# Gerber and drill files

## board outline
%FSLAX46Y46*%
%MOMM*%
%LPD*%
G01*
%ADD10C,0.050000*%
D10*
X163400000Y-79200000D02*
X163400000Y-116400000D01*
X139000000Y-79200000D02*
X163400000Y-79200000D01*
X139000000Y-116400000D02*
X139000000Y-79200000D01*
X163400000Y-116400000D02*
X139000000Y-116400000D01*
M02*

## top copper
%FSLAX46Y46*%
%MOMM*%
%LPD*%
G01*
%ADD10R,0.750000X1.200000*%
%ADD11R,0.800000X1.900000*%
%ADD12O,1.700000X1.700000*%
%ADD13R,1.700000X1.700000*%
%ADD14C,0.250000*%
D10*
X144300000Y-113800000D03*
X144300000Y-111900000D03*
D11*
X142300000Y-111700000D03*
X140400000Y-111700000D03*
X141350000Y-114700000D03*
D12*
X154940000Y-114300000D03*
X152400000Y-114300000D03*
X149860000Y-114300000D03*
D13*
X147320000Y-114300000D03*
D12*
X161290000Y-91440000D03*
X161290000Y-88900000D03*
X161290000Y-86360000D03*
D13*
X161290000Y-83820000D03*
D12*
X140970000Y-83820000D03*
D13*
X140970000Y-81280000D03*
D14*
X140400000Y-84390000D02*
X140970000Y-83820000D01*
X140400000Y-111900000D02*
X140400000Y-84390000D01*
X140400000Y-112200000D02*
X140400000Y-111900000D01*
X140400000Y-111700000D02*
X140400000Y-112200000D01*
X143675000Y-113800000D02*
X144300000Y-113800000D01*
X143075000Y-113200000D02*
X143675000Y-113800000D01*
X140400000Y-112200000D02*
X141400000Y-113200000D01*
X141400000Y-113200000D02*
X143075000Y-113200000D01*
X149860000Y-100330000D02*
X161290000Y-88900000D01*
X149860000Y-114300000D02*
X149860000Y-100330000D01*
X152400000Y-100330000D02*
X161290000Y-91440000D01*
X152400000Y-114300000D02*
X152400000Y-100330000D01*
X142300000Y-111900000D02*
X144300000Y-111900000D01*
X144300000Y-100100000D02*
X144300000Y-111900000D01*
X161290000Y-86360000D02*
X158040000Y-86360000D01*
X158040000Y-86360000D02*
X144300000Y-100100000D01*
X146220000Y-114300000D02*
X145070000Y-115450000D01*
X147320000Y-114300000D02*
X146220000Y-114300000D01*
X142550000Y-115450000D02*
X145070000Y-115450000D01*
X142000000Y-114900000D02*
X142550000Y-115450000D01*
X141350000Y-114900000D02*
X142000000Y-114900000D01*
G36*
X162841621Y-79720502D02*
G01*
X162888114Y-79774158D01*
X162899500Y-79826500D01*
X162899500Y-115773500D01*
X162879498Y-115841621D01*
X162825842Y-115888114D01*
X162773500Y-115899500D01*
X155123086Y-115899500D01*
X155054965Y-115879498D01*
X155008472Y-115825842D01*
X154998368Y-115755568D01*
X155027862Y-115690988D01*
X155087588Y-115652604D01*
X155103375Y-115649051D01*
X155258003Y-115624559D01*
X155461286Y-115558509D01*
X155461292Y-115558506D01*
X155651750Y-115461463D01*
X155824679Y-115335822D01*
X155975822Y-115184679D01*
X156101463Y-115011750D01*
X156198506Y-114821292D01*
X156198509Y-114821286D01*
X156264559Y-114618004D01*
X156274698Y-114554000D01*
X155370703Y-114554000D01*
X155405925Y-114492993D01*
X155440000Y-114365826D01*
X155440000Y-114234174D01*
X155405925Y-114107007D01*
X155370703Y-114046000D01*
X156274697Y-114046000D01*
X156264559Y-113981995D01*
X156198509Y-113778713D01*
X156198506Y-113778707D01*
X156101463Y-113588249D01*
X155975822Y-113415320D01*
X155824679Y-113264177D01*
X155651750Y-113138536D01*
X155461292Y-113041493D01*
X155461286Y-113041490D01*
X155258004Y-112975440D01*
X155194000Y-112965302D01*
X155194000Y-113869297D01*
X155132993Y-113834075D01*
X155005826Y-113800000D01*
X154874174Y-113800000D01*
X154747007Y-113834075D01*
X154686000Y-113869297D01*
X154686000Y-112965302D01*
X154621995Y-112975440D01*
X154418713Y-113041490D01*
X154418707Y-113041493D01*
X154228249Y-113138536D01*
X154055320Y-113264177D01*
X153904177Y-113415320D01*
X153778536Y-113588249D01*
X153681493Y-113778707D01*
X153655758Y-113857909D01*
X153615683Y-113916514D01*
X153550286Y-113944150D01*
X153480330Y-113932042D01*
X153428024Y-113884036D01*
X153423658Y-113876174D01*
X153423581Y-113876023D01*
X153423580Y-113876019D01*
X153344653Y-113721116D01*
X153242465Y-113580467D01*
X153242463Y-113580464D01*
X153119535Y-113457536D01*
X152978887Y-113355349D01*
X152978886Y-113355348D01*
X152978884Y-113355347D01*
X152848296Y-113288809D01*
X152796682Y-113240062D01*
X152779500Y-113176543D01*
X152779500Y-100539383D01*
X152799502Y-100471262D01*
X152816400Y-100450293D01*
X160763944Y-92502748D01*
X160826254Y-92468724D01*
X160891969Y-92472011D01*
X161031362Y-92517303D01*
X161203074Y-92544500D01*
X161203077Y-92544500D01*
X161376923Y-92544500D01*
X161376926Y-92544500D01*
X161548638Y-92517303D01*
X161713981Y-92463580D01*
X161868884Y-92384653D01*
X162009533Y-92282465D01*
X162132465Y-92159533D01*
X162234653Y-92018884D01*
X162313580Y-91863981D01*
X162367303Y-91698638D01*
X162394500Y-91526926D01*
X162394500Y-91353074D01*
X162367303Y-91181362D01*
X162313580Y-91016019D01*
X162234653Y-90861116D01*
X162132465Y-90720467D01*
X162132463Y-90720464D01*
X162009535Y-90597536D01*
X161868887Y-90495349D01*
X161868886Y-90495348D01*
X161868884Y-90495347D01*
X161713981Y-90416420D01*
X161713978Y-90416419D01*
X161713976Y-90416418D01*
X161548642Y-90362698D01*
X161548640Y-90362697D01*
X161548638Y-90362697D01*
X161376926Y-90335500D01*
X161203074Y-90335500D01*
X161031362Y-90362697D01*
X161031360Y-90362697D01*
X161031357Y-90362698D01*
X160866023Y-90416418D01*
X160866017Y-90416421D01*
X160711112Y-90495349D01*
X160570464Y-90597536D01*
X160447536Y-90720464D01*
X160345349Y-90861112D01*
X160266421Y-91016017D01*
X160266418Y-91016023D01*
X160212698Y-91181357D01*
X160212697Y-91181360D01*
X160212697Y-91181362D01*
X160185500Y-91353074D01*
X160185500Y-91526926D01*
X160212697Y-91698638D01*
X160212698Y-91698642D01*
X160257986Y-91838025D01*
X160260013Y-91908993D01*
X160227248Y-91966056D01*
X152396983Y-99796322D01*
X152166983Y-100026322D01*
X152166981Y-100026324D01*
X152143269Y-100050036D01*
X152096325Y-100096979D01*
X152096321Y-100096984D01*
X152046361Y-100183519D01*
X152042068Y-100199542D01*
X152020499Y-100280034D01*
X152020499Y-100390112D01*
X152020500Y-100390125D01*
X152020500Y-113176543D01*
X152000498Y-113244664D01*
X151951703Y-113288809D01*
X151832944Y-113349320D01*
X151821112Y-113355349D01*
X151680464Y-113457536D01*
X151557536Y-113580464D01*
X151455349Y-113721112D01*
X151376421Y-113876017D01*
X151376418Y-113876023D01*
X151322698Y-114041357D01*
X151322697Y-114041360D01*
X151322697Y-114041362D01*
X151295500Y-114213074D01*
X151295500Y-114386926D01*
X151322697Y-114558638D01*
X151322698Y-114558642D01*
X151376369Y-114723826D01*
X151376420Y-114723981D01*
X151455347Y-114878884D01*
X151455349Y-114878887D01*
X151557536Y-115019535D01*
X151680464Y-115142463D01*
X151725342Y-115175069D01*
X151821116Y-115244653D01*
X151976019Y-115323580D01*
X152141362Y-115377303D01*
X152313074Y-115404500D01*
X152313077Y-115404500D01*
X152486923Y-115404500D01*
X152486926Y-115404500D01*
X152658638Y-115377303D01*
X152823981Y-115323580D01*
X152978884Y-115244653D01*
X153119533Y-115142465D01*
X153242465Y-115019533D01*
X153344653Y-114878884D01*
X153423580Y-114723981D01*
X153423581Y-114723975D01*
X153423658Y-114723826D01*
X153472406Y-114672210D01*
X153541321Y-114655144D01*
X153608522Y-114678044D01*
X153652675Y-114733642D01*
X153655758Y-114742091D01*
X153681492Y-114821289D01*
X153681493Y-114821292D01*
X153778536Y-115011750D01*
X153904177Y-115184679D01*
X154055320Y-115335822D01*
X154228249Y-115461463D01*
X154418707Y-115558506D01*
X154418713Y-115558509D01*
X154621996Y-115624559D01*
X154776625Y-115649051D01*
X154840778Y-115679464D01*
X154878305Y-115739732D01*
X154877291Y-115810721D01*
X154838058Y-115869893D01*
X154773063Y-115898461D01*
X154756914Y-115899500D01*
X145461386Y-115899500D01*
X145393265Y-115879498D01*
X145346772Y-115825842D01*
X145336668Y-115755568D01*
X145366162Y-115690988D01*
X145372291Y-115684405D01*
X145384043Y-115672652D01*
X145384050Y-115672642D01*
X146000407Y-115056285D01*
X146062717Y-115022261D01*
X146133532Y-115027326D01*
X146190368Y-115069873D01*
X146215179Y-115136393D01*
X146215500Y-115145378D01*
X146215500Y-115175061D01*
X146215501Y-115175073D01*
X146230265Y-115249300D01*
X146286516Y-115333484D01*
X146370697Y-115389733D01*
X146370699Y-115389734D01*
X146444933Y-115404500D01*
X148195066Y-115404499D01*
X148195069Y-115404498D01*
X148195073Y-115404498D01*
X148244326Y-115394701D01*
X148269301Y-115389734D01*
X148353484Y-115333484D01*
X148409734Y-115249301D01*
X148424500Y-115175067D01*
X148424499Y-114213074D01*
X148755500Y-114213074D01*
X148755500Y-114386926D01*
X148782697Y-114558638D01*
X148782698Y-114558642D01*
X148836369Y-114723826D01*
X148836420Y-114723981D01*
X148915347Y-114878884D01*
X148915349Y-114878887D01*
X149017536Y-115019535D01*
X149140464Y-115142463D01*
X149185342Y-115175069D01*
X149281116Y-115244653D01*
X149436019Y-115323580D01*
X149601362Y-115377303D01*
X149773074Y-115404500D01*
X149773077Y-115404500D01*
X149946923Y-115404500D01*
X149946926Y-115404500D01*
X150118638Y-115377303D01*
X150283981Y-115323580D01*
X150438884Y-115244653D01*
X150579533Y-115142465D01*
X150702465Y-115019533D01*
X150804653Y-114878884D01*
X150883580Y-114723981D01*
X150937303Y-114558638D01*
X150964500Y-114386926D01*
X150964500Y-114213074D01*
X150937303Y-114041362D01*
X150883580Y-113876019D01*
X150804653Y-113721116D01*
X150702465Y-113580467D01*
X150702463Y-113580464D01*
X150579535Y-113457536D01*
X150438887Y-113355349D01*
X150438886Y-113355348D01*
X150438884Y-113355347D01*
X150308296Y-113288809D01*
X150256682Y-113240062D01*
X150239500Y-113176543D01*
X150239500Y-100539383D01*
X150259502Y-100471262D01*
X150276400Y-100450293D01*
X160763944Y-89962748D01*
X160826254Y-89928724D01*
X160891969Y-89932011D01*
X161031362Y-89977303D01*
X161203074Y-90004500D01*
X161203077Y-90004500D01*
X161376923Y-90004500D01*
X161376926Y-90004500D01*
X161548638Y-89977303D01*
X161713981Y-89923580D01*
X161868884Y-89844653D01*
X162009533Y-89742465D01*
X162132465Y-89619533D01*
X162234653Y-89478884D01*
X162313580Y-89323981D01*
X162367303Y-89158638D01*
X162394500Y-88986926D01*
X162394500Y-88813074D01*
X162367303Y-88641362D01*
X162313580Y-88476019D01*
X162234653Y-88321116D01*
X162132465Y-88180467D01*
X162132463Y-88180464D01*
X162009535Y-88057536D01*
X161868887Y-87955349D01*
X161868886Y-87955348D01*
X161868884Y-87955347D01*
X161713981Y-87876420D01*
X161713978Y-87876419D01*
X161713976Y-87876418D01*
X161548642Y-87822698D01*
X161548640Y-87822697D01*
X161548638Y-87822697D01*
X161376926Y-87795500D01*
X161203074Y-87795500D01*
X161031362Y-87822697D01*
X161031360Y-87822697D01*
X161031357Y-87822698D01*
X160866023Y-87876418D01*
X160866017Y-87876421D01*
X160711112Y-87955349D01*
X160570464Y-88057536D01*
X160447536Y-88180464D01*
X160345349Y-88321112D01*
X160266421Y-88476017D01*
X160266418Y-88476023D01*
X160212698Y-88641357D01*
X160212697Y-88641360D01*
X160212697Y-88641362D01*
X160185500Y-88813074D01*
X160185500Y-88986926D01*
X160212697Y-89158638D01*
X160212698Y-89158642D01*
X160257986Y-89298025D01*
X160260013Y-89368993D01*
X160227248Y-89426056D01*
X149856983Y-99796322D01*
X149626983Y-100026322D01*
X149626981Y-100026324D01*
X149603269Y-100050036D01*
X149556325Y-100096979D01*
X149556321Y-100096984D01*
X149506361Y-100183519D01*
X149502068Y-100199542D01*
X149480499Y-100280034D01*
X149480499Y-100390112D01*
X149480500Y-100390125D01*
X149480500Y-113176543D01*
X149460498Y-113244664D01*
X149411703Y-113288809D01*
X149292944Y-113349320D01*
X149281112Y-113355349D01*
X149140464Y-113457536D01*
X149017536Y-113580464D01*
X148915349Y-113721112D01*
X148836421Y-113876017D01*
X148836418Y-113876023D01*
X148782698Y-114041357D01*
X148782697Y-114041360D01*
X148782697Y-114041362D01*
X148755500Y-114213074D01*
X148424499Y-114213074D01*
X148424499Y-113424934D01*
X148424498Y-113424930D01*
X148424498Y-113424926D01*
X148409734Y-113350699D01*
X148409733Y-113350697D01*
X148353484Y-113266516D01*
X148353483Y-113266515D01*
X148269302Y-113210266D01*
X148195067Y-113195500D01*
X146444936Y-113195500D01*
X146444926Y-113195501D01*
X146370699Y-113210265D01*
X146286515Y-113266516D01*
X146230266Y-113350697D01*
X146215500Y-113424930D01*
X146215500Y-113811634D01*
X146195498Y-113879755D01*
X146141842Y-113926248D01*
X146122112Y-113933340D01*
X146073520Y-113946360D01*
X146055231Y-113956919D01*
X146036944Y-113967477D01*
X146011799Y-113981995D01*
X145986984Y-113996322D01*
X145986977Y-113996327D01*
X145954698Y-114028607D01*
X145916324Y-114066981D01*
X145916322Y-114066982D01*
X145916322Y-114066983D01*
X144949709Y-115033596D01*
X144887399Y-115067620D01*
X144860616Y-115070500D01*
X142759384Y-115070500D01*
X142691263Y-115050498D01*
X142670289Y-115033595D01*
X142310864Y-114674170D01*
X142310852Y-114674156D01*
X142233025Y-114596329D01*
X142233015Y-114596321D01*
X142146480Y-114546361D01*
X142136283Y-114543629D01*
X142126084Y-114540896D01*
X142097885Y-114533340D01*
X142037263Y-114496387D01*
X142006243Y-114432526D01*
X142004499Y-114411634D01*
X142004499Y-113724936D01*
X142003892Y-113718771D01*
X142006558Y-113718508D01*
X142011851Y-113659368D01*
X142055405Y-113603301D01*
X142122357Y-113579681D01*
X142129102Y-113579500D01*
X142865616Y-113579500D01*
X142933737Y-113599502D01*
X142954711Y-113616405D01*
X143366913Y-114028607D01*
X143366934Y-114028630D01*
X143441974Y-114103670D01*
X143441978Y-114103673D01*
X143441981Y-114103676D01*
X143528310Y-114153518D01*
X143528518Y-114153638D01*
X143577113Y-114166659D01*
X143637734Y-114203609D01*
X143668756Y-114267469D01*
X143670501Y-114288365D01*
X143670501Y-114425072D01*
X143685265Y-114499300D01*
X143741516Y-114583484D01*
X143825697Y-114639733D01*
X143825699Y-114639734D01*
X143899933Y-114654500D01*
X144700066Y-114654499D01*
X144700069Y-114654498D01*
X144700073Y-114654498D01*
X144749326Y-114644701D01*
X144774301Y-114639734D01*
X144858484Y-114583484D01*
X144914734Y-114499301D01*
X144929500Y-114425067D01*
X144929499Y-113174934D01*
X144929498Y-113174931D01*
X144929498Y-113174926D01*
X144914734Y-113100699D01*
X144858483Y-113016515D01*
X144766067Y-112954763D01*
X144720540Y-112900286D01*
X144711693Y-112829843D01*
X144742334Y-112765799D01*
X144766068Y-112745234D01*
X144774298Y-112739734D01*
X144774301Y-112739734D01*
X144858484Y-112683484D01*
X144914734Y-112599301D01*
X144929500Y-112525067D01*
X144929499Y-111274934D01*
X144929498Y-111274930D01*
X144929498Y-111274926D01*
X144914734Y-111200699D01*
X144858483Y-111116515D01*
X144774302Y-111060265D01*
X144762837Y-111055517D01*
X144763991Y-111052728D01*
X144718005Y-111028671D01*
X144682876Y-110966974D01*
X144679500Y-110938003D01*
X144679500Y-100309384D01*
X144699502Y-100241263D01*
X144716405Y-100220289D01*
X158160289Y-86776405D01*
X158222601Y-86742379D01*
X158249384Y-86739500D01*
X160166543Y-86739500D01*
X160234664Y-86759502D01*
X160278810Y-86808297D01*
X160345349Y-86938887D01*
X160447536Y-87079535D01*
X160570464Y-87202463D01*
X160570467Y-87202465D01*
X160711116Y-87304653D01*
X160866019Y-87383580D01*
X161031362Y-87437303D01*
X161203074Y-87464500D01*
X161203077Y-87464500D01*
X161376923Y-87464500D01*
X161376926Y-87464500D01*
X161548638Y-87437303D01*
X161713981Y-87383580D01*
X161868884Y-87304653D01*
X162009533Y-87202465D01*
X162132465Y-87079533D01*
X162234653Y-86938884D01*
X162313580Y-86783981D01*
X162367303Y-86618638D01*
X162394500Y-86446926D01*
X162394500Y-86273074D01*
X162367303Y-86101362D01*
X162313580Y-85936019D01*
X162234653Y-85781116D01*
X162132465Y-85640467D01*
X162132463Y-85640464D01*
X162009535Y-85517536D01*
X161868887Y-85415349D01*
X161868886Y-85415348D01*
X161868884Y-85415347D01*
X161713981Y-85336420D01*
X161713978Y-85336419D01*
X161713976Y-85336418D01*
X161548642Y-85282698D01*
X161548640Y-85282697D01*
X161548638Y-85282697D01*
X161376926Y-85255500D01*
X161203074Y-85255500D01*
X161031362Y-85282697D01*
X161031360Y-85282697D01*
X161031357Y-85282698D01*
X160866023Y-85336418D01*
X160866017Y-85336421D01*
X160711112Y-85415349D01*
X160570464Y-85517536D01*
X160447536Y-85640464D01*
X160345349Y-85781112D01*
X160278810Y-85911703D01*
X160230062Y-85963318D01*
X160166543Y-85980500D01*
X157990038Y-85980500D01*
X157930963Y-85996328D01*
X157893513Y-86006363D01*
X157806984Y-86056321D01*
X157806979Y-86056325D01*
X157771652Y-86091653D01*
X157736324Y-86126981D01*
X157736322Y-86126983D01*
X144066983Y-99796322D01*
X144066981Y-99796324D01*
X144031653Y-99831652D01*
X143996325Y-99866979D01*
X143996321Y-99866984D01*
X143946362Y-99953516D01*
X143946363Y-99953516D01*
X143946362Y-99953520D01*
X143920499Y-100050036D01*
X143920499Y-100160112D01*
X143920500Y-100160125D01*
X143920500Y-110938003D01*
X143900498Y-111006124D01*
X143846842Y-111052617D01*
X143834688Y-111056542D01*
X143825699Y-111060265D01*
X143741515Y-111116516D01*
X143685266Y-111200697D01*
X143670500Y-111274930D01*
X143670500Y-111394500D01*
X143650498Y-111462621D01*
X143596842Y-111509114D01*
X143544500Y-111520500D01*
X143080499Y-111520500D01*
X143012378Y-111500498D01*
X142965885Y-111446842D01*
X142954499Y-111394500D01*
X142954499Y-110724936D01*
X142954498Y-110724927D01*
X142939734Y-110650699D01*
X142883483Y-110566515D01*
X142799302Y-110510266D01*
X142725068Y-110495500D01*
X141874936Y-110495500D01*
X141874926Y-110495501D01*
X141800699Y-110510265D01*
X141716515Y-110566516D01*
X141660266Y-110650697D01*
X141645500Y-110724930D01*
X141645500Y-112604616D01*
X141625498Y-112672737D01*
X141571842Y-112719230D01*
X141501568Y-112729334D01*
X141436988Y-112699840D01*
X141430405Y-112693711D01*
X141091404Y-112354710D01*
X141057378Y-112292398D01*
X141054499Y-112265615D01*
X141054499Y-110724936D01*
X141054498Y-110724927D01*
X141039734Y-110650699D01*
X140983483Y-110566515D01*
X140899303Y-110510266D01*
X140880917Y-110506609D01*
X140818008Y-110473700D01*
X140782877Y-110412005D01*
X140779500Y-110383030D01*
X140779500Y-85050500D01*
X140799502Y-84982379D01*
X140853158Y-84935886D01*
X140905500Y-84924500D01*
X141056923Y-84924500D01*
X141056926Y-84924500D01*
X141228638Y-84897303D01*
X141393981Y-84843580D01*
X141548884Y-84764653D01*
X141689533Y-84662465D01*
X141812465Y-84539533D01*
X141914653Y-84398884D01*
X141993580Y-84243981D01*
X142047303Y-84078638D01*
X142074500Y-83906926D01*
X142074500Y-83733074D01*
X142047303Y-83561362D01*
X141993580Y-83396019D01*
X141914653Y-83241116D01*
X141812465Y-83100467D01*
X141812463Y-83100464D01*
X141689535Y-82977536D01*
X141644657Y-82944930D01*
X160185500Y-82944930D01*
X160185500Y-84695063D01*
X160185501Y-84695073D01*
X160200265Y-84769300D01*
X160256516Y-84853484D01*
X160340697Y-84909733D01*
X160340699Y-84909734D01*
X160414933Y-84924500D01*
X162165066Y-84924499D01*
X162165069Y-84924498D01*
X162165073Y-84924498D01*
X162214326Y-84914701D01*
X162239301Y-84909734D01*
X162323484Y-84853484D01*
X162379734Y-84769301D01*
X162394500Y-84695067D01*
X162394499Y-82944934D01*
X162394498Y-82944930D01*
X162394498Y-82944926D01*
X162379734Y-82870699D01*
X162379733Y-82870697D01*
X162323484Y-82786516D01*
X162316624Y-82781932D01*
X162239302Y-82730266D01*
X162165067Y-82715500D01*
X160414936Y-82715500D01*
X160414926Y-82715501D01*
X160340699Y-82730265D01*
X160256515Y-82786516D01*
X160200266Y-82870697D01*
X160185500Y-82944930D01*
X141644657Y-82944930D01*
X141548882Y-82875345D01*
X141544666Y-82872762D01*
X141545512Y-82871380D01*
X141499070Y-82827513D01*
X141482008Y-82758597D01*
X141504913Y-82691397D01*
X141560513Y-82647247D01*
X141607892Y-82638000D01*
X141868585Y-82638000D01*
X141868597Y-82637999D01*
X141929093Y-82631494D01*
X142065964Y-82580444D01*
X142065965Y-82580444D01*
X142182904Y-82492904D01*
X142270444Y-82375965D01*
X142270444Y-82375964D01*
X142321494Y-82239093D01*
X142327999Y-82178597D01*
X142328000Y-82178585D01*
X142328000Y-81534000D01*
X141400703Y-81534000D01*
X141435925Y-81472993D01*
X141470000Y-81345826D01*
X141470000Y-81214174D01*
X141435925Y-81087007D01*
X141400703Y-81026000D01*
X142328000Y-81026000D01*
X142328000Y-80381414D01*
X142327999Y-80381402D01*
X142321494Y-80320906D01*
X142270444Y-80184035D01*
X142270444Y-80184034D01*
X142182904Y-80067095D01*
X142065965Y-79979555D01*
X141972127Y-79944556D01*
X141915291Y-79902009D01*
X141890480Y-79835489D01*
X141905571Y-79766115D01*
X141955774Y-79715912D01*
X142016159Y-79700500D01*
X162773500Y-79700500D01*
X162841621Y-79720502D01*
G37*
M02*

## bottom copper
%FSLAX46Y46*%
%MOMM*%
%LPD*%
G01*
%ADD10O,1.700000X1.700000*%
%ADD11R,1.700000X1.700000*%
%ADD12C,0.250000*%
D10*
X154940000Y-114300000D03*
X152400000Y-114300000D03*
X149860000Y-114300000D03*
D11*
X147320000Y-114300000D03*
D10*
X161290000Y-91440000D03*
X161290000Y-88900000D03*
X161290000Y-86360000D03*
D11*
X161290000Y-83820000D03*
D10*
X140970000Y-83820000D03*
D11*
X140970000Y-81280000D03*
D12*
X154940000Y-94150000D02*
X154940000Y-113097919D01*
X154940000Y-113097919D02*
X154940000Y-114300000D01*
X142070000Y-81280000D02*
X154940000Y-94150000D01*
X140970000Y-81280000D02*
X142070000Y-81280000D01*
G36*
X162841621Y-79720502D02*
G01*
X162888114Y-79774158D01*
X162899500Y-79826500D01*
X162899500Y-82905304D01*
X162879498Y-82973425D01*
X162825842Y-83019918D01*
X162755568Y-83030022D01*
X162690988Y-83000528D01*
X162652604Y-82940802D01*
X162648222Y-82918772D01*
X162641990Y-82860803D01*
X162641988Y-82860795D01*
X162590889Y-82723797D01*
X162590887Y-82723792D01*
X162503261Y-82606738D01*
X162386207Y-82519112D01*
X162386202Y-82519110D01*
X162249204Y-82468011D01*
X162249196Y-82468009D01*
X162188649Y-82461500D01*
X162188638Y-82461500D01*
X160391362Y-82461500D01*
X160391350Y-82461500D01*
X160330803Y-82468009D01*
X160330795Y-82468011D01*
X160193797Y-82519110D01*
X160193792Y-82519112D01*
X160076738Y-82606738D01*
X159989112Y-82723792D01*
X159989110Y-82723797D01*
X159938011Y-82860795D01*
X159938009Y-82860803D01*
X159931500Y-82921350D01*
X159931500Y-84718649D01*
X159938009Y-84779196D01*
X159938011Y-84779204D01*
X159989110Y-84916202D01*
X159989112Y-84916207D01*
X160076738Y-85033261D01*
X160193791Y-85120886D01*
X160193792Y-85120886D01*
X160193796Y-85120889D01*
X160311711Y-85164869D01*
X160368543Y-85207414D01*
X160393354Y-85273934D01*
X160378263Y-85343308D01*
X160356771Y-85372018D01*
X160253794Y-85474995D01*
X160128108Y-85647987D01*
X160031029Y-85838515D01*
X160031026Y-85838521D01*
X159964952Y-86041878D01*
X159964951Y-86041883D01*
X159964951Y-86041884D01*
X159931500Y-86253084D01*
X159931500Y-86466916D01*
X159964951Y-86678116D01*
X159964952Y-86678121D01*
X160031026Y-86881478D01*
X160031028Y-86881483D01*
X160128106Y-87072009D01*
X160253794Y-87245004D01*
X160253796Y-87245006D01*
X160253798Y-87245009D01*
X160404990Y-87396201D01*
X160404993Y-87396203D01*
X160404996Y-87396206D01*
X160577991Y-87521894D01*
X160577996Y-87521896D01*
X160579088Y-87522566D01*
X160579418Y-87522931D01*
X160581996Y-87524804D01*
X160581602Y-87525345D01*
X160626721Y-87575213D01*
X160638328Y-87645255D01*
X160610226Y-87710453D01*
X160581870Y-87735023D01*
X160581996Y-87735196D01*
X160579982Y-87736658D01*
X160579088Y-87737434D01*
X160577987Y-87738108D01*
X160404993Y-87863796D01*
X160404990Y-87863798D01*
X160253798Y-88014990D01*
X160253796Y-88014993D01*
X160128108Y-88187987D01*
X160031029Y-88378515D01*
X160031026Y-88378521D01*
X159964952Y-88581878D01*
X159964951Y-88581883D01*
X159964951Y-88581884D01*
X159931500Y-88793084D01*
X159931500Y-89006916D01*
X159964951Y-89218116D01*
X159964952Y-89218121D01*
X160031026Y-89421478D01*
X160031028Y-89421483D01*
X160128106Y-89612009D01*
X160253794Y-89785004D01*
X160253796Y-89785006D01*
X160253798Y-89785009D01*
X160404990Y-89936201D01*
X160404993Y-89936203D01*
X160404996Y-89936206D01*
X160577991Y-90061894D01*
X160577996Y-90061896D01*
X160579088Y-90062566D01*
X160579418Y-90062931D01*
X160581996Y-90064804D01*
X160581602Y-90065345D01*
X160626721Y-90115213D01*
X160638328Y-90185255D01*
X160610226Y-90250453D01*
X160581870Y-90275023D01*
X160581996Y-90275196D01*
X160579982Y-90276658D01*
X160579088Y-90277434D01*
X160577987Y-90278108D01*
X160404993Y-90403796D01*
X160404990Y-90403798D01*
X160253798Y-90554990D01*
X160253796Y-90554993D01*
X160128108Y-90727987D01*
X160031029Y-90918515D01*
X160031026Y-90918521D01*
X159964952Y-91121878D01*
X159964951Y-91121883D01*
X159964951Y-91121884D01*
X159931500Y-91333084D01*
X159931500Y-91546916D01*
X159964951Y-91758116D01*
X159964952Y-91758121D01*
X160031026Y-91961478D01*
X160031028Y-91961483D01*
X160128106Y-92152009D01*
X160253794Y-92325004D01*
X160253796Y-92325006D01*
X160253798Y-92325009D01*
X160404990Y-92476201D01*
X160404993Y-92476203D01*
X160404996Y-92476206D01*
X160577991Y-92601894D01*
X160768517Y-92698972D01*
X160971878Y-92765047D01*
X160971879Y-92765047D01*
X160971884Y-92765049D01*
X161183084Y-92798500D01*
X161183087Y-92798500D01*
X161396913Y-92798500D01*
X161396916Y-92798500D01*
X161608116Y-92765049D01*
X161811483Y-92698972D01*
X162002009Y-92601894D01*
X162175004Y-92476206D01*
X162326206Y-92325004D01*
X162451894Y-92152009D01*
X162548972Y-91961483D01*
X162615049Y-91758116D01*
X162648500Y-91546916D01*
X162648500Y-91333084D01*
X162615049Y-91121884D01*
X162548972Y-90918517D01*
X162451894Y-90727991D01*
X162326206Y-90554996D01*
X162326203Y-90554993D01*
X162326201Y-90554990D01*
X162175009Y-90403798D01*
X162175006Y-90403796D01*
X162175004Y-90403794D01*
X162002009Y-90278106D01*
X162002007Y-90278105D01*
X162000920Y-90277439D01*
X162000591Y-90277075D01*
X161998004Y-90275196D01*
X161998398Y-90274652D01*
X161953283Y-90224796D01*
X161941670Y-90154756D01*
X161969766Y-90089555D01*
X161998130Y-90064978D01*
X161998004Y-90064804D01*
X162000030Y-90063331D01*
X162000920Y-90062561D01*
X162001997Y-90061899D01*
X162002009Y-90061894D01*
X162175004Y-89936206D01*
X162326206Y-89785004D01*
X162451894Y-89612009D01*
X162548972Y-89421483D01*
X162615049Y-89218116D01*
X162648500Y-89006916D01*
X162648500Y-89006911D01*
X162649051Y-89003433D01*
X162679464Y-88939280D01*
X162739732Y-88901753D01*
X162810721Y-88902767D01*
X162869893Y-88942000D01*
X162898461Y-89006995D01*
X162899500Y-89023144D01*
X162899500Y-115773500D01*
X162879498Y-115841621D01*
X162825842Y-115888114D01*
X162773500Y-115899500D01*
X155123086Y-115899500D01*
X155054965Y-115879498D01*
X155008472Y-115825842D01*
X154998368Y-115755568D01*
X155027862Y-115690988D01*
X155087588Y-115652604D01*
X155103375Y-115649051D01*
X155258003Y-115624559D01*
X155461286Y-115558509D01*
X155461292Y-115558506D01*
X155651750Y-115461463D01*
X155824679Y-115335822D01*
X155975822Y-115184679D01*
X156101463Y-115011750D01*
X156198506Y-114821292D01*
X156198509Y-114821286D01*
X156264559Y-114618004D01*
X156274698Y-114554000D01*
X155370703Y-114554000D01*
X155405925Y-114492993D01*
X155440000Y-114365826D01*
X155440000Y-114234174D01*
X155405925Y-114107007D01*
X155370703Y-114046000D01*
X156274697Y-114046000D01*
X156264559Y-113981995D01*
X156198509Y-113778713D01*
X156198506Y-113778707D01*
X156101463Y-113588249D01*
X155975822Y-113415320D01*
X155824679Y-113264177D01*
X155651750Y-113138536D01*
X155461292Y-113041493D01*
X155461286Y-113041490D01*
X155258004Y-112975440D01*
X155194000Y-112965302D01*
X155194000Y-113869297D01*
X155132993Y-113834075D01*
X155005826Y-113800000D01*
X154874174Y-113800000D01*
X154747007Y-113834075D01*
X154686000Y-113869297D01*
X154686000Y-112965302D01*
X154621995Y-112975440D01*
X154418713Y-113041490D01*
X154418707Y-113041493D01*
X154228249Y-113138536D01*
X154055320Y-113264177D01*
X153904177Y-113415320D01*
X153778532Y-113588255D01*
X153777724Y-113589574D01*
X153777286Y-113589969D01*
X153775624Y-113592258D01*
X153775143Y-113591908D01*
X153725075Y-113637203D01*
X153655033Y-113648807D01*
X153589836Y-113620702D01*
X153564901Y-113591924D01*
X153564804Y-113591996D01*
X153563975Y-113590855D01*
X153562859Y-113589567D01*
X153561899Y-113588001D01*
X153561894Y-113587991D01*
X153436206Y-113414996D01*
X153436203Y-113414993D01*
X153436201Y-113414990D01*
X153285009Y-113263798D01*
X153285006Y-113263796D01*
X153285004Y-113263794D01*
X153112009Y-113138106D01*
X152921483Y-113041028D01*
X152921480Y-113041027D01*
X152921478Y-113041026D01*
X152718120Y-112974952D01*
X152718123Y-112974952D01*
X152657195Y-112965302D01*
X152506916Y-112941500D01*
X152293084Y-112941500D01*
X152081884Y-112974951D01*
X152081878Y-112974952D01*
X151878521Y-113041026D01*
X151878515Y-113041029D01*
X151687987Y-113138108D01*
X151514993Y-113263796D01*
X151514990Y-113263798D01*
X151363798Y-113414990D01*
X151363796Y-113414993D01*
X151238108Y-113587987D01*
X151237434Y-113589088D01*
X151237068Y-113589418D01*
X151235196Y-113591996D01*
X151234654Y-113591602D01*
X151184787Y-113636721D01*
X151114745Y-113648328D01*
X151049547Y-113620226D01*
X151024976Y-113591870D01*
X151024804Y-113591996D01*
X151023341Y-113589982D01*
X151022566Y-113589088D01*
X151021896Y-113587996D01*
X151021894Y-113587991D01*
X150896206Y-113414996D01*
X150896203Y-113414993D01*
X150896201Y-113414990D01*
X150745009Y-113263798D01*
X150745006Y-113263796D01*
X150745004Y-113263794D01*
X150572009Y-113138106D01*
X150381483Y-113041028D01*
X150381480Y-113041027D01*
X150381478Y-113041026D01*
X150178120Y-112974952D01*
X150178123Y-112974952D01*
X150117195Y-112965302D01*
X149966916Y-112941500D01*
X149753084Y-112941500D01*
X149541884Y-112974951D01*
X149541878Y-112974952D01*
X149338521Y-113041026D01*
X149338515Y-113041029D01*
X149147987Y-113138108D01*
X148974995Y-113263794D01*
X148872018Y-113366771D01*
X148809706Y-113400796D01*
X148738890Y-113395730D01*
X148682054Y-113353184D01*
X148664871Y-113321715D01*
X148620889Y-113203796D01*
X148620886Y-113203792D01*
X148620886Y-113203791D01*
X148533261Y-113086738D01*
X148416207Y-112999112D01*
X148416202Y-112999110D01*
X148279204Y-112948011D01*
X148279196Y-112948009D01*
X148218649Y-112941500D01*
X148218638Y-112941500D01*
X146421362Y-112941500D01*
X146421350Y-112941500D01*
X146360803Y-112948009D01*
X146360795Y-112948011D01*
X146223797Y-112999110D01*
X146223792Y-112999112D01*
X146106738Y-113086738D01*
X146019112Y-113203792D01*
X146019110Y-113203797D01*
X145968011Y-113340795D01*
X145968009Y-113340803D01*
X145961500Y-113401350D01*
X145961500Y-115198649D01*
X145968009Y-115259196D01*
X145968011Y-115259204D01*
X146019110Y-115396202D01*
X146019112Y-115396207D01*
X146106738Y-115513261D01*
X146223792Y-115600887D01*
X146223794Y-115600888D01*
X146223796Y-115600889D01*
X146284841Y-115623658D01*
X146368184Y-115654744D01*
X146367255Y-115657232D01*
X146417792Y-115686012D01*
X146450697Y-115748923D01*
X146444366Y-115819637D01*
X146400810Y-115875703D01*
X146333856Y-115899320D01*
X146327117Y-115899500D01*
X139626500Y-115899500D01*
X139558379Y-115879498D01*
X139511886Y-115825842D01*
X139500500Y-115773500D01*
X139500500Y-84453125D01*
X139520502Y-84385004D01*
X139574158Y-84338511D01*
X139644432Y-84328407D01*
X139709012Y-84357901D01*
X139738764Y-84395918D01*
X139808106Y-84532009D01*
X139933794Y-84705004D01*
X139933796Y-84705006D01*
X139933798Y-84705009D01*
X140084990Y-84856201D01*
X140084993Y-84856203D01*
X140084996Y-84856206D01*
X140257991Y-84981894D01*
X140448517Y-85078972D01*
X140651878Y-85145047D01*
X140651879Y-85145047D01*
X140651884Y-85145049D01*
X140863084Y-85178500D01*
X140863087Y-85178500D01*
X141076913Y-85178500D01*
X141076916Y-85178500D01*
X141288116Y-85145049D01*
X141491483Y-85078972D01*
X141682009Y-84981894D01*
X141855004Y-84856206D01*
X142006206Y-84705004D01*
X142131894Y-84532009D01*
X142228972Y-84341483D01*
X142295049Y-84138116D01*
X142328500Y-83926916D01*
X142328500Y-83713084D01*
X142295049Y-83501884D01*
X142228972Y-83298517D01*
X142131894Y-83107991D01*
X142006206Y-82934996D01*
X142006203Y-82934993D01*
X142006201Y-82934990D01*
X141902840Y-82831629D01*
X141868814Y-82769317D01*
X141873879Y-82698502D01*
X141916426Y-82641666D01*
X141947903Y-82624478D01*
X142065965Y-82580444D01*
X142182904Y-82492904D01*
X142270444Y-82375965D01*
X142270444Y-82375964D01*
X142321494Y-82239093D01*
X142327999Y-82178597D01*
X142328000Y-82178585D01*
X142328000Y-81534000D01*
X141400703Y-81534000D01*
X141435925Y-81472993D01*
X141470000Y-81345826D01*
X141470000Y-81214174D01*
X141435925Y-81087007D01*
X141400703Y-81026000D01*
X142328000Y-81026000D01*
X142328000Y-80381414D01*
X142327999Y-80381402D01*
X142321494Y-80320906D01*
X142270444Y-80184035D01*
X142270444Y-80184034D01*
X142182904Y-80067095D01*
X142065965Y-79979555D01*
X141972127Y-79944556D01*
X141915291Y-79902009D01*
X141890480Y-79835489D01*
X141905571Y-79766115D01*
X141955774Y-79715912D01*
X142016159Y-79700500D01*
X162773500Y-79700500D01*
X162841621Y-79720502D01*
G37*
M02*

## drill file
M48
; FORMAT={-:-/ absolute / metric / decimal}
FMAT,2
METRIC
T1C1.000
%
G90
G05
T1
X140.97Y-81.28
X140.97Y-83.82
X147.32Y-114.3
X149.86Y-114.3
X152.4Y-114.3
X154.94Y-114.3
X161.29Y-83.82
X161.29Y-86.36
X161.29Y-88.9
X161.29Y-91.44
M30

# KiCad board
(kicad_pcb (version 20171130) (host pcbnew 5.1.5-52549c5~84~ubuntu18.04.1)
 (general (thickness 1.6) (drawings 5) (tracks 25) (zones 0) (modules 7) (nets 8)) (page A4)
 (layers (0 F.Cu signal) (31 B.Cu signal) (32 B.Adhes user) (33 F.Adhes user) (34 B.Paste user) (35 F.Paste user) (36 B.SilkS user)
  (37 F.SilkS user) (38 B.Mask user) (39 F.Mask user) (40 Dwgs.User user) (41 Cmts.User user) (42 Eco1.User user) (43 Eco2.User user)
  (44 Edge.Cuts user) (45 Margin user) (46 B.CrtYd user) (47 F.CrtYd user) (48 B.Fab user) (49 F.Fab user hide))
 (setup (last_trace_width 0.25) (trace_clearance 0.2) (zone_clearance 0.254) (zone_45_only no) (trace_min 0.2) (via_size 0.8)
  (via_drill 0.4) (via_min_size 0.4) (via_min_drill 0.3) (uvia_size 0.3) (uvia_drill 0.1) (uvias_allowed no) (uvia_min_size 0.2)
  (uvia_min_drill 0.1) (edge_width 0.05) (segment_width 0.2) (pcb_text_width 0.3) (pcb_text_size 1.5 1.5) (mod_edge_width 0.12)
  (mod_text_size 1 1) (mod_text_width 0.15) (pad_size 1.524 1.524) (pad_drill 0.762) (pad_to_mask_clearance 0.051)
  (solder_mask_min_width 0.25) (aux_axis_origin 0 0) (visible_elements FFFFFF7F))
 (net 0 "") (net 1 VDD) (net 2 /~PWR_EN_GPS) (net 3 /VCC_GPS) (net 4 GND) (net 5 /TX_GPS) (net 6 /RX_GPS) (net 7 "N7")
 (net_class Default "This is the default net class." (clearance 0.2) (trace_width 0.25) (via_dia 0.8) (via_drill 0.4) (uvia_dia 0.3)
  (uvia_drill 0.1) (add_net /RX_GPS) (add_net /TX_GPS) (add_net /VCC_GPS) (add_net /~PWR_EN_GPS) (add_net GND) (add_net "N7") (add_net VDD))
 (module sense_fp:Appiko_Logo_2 (layer F.Cu) (at 148.65 99.3)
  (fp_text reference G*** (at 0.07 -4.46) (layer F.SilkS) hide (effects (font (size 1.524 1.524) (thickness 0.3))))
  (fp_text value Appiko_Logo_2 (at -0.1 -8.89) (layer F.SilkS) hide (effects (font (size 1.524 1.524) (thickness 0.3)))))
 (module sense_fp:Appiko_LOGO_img (layer F.Cu) (at 150.5 88.4)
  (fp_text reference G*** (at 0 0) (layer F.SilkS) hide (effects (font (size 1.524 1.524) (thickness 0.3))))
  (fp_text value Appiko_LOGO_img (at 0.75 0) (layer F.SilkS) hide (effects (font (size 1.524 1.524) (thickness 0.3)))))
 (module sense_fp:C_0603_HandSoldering (layer F.Cu) (at 144.3 112.85 90)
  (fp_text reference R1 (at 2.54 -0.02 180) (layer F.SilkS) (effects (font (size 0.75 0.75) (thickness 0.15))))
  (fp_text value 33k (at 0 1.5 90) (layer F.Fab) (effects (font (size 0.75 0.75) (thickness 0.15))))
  (pad 1 smd rect (at -0.95 0 90) (size 1.2 0.75) (layers F.Cu F.Paste F.Mask) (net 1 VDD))
  (pad 2 smd rect (at 0.95 0 90) (size 1.2 0.75) (layers F.Cu F.Paste F.Mask) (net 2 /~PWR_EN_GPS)))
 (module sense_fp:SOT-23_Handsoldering (layer F.Cu) (at 141.35 113.2 270)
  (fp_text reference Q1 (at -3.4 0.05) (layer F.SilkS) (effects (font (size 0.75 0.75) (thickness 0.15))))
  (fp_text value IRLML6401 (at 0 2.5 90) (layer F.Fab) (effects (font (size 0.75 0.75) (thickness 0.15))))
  (pad 1 smd rect (at -1.5 -0.95 270) (size 1.9 0.8) (layers F.Cu F.Paste F.Mask) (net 2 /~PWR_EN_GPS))
  (pad 2 smd rect (at -1.5 0.95 270) (size 1.9 0.8) (layers F.Cu F.Paste F.Mask) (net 1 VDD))
  (pad 3 smd rect (at 1.5 0 270) (size 1.9 0.8) (layers F.Cu F.Paste F.Mask) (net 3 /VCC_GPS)))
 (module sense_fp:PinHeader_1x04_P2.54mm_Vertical (layer F.Cu) (at 147.32 114.3 90)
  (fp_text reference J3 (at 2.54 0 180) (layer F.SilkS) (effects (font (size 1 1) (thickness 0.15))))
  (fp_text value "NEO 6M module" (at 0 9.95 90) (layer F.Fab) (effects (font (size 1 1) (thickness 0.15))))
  (pad 4 thru_hole oval (at 0 7.62 90) (size 1.7 1.7) (drill 1) (layers *.Cu *.Mask) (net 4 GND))
  (pad 3 thru_hole oval (at 0 5.08 90) (size 1.7 1.7) (drill 1) (layers *.Cu *.Mask) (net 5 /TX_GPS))
  (pad 2 thru_hole oval (at 0 2.54 90) (size 1.7 1.7) (drill 1) (layers *.Cu *.Mask) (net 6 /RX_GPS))
  (pad 1 thru_hole rect (at 0 0 90) (size 1.7 1.7) (drill 1) (layers *.Cu *.Mask) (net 3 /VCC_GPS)))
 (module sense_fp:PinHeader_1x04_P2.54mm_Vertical (layer F.Cu) (at 161.29 83.82)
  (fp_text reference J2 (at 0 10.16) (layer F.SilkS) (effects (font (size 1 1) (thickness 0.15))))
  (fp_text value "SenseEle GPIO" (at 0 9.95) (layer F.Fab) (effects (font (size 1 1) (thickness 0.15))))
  (pad 4 thru_hole oval (at 0 7.62) (size 1.7 1.7) (drill 1) (layers *.Cu *.Mask) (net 5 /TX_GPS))
  (pad 3 thru_hole oval (at 0 5.08) (size 1.7 1.7) (drill 1) (layers *.Cu *.Mask) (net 6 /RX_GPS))
  (pad 2 thru_hole oval (at 0 2.54) (size 1.7 1.7) (drill 1) (layers *.Cu *.Mask) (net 2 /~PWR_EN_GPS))
  (pad 1 thru_hole rect (at 0 0) (size 1.7 1.7) (drill 1) (layers *.Cu *.Mask) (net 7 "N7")))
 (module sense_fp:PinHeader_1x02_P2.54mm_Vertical (layer F.Cu) (at 140.97 81.28)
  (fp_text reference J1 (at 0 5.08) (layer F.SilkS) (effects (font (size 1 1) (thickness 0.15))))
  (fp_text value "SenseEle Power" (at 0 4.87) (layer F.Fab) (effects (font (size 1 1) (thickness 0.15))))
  (pad 2 thru_hole oval (at 0 2.54) (size 1.7 1.7) (drill 1) (layers *.Cu *.Mask) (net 1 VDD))
  (pad 1 thru_hole rect (at 0 0) (size 1.7 1.7) (drill 1) (layers *.Cu *.Mask) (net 4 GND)))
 (gr_line (start 163.4 79.2) (end 163.4 116.4) (layer Edge.Cuts) (width 0.05))
 (gr_line (start 139 79.2) (end 163.4 79.2) (layer Edge.Cuts) (width 0.05))
 (gr_line (start 139 116.4) (end 139 79.2) (layer Edge.Cuts) (width 0.05))
 (gr_line (start 163.4 116.4) (end 139 116.4) (layer Edge.Cuts) (width 0.05))
 (segment (start 140.4 84.39) (end 140.97 83.82) (width 0.25) (layer F.Cu) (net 1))
 (segment (start 140.4 111.9) (end 140.4 84.39) (width 0.25) (layer F.Cu) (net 1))
 (segment (start 140.4 112.2) (end 140.4 111.9) (width 0.25) (layer F.Cu) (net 1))
 (segment (start 140.4 111.7) (end 140.4 112.2) (width 0.25) (layer F.Cu) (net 1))
 (segment (start 143.675 113.8) (end 144.3 113.8) (width 0.25) (layer F.Cu) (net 1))
 (segment (start 143.075 113.2) (end 143.675 113.8) (width 0.25) (layer F.Cu) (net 1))
 (segment (start 140.4 112.2) (end 141.4 113.2) (width 0.25) (layer F.Cu) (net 1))
 (segment (start 141.4 113.2) (end 143.075 113.2) (width 0.25) (layer F.Cu) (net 1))
 (segment (start 154.94 94.15) (end 154.94 113.097919) (width 0.25) (layer B.Cu) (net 4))
 (segment (start 154.94 113.097919) (end 154.94 114.3) (width 0.25) (layer B.Cu) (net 4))
 (segment (start 142.07 81.28) (end 154.94 94.15) (width 0.25) (layer B.Cu) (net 4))
 (segment (start 140.97 81.28) (end 142.07 81.28) (width 0.25) (layer B.Cu) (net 4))
 (segment (start 149.86 100.33) (end 161.29 88.9) (width 0.25) (layer F.Cu) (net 6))
 (segment (start 149.86 114.3) (end 149.86 100.33) (width 0.25) (layer F.Cu) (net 6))
 (segment (start 152.4 100.33) (end 161.29 91.44) (width 0.25) (layer F.Cu) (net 5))
 (segment (start 152.4 114.3) (end 152.4 100.33) (width 0.25) (layer F.Cu) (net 5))
 (segment (start 142.3 111.9) (end 144.3 111.9) (width 0.25) (layer F.Cu) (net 2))
 (segment (start 144.3 100.1) (end 144.3 111.9) (width 0.25) (layer F.Cu) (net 2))
 (segment (start 161.29 86.36) (end 158.04 86.36) (width 0.25) (layer F.Cu) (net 2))
 (segment (start 158.04 86.36) (end 144.3 100.1) (width 0.25) (layer F.Cu) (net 2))
 (segment (start 146.22 114.3) (end 145.07 115.45) (width 0.25) (layer F.Cu) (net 3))
 (segment (start 147.32 114.3) (end 146.22 114.3) (width 0.25) (layer F.Cu) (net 3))
 (segment (start 142.55 115.45) (end 145.07 115.45) (width 0.25) (layer F.Cu) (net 3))
 (segment (start 142 114.9) (end 142.55 115.45) (width 0.25) (layer F.Cu) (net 3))
 (segment (start 141.35 114.9) (end 142 114.9) (width 0.25) (layer F.Cu) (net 3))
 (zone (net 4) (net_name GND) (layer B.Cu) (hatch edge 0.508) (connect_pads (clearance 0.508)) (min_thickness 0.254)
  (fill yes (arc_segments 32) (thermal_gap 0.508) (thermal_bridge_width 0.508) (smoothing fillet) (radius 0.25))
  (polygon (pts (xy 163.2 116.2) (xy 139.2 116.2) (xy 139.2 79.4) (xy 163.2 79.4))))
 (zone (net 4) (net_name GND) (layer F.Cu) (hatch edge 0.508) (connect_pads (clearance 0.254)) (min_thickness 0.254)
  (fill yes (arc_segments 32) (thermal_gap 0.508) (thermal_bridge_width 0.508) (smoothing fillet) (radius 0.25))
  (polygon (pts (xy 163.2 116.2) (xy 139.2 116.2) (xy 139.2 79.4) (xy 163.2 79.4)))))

